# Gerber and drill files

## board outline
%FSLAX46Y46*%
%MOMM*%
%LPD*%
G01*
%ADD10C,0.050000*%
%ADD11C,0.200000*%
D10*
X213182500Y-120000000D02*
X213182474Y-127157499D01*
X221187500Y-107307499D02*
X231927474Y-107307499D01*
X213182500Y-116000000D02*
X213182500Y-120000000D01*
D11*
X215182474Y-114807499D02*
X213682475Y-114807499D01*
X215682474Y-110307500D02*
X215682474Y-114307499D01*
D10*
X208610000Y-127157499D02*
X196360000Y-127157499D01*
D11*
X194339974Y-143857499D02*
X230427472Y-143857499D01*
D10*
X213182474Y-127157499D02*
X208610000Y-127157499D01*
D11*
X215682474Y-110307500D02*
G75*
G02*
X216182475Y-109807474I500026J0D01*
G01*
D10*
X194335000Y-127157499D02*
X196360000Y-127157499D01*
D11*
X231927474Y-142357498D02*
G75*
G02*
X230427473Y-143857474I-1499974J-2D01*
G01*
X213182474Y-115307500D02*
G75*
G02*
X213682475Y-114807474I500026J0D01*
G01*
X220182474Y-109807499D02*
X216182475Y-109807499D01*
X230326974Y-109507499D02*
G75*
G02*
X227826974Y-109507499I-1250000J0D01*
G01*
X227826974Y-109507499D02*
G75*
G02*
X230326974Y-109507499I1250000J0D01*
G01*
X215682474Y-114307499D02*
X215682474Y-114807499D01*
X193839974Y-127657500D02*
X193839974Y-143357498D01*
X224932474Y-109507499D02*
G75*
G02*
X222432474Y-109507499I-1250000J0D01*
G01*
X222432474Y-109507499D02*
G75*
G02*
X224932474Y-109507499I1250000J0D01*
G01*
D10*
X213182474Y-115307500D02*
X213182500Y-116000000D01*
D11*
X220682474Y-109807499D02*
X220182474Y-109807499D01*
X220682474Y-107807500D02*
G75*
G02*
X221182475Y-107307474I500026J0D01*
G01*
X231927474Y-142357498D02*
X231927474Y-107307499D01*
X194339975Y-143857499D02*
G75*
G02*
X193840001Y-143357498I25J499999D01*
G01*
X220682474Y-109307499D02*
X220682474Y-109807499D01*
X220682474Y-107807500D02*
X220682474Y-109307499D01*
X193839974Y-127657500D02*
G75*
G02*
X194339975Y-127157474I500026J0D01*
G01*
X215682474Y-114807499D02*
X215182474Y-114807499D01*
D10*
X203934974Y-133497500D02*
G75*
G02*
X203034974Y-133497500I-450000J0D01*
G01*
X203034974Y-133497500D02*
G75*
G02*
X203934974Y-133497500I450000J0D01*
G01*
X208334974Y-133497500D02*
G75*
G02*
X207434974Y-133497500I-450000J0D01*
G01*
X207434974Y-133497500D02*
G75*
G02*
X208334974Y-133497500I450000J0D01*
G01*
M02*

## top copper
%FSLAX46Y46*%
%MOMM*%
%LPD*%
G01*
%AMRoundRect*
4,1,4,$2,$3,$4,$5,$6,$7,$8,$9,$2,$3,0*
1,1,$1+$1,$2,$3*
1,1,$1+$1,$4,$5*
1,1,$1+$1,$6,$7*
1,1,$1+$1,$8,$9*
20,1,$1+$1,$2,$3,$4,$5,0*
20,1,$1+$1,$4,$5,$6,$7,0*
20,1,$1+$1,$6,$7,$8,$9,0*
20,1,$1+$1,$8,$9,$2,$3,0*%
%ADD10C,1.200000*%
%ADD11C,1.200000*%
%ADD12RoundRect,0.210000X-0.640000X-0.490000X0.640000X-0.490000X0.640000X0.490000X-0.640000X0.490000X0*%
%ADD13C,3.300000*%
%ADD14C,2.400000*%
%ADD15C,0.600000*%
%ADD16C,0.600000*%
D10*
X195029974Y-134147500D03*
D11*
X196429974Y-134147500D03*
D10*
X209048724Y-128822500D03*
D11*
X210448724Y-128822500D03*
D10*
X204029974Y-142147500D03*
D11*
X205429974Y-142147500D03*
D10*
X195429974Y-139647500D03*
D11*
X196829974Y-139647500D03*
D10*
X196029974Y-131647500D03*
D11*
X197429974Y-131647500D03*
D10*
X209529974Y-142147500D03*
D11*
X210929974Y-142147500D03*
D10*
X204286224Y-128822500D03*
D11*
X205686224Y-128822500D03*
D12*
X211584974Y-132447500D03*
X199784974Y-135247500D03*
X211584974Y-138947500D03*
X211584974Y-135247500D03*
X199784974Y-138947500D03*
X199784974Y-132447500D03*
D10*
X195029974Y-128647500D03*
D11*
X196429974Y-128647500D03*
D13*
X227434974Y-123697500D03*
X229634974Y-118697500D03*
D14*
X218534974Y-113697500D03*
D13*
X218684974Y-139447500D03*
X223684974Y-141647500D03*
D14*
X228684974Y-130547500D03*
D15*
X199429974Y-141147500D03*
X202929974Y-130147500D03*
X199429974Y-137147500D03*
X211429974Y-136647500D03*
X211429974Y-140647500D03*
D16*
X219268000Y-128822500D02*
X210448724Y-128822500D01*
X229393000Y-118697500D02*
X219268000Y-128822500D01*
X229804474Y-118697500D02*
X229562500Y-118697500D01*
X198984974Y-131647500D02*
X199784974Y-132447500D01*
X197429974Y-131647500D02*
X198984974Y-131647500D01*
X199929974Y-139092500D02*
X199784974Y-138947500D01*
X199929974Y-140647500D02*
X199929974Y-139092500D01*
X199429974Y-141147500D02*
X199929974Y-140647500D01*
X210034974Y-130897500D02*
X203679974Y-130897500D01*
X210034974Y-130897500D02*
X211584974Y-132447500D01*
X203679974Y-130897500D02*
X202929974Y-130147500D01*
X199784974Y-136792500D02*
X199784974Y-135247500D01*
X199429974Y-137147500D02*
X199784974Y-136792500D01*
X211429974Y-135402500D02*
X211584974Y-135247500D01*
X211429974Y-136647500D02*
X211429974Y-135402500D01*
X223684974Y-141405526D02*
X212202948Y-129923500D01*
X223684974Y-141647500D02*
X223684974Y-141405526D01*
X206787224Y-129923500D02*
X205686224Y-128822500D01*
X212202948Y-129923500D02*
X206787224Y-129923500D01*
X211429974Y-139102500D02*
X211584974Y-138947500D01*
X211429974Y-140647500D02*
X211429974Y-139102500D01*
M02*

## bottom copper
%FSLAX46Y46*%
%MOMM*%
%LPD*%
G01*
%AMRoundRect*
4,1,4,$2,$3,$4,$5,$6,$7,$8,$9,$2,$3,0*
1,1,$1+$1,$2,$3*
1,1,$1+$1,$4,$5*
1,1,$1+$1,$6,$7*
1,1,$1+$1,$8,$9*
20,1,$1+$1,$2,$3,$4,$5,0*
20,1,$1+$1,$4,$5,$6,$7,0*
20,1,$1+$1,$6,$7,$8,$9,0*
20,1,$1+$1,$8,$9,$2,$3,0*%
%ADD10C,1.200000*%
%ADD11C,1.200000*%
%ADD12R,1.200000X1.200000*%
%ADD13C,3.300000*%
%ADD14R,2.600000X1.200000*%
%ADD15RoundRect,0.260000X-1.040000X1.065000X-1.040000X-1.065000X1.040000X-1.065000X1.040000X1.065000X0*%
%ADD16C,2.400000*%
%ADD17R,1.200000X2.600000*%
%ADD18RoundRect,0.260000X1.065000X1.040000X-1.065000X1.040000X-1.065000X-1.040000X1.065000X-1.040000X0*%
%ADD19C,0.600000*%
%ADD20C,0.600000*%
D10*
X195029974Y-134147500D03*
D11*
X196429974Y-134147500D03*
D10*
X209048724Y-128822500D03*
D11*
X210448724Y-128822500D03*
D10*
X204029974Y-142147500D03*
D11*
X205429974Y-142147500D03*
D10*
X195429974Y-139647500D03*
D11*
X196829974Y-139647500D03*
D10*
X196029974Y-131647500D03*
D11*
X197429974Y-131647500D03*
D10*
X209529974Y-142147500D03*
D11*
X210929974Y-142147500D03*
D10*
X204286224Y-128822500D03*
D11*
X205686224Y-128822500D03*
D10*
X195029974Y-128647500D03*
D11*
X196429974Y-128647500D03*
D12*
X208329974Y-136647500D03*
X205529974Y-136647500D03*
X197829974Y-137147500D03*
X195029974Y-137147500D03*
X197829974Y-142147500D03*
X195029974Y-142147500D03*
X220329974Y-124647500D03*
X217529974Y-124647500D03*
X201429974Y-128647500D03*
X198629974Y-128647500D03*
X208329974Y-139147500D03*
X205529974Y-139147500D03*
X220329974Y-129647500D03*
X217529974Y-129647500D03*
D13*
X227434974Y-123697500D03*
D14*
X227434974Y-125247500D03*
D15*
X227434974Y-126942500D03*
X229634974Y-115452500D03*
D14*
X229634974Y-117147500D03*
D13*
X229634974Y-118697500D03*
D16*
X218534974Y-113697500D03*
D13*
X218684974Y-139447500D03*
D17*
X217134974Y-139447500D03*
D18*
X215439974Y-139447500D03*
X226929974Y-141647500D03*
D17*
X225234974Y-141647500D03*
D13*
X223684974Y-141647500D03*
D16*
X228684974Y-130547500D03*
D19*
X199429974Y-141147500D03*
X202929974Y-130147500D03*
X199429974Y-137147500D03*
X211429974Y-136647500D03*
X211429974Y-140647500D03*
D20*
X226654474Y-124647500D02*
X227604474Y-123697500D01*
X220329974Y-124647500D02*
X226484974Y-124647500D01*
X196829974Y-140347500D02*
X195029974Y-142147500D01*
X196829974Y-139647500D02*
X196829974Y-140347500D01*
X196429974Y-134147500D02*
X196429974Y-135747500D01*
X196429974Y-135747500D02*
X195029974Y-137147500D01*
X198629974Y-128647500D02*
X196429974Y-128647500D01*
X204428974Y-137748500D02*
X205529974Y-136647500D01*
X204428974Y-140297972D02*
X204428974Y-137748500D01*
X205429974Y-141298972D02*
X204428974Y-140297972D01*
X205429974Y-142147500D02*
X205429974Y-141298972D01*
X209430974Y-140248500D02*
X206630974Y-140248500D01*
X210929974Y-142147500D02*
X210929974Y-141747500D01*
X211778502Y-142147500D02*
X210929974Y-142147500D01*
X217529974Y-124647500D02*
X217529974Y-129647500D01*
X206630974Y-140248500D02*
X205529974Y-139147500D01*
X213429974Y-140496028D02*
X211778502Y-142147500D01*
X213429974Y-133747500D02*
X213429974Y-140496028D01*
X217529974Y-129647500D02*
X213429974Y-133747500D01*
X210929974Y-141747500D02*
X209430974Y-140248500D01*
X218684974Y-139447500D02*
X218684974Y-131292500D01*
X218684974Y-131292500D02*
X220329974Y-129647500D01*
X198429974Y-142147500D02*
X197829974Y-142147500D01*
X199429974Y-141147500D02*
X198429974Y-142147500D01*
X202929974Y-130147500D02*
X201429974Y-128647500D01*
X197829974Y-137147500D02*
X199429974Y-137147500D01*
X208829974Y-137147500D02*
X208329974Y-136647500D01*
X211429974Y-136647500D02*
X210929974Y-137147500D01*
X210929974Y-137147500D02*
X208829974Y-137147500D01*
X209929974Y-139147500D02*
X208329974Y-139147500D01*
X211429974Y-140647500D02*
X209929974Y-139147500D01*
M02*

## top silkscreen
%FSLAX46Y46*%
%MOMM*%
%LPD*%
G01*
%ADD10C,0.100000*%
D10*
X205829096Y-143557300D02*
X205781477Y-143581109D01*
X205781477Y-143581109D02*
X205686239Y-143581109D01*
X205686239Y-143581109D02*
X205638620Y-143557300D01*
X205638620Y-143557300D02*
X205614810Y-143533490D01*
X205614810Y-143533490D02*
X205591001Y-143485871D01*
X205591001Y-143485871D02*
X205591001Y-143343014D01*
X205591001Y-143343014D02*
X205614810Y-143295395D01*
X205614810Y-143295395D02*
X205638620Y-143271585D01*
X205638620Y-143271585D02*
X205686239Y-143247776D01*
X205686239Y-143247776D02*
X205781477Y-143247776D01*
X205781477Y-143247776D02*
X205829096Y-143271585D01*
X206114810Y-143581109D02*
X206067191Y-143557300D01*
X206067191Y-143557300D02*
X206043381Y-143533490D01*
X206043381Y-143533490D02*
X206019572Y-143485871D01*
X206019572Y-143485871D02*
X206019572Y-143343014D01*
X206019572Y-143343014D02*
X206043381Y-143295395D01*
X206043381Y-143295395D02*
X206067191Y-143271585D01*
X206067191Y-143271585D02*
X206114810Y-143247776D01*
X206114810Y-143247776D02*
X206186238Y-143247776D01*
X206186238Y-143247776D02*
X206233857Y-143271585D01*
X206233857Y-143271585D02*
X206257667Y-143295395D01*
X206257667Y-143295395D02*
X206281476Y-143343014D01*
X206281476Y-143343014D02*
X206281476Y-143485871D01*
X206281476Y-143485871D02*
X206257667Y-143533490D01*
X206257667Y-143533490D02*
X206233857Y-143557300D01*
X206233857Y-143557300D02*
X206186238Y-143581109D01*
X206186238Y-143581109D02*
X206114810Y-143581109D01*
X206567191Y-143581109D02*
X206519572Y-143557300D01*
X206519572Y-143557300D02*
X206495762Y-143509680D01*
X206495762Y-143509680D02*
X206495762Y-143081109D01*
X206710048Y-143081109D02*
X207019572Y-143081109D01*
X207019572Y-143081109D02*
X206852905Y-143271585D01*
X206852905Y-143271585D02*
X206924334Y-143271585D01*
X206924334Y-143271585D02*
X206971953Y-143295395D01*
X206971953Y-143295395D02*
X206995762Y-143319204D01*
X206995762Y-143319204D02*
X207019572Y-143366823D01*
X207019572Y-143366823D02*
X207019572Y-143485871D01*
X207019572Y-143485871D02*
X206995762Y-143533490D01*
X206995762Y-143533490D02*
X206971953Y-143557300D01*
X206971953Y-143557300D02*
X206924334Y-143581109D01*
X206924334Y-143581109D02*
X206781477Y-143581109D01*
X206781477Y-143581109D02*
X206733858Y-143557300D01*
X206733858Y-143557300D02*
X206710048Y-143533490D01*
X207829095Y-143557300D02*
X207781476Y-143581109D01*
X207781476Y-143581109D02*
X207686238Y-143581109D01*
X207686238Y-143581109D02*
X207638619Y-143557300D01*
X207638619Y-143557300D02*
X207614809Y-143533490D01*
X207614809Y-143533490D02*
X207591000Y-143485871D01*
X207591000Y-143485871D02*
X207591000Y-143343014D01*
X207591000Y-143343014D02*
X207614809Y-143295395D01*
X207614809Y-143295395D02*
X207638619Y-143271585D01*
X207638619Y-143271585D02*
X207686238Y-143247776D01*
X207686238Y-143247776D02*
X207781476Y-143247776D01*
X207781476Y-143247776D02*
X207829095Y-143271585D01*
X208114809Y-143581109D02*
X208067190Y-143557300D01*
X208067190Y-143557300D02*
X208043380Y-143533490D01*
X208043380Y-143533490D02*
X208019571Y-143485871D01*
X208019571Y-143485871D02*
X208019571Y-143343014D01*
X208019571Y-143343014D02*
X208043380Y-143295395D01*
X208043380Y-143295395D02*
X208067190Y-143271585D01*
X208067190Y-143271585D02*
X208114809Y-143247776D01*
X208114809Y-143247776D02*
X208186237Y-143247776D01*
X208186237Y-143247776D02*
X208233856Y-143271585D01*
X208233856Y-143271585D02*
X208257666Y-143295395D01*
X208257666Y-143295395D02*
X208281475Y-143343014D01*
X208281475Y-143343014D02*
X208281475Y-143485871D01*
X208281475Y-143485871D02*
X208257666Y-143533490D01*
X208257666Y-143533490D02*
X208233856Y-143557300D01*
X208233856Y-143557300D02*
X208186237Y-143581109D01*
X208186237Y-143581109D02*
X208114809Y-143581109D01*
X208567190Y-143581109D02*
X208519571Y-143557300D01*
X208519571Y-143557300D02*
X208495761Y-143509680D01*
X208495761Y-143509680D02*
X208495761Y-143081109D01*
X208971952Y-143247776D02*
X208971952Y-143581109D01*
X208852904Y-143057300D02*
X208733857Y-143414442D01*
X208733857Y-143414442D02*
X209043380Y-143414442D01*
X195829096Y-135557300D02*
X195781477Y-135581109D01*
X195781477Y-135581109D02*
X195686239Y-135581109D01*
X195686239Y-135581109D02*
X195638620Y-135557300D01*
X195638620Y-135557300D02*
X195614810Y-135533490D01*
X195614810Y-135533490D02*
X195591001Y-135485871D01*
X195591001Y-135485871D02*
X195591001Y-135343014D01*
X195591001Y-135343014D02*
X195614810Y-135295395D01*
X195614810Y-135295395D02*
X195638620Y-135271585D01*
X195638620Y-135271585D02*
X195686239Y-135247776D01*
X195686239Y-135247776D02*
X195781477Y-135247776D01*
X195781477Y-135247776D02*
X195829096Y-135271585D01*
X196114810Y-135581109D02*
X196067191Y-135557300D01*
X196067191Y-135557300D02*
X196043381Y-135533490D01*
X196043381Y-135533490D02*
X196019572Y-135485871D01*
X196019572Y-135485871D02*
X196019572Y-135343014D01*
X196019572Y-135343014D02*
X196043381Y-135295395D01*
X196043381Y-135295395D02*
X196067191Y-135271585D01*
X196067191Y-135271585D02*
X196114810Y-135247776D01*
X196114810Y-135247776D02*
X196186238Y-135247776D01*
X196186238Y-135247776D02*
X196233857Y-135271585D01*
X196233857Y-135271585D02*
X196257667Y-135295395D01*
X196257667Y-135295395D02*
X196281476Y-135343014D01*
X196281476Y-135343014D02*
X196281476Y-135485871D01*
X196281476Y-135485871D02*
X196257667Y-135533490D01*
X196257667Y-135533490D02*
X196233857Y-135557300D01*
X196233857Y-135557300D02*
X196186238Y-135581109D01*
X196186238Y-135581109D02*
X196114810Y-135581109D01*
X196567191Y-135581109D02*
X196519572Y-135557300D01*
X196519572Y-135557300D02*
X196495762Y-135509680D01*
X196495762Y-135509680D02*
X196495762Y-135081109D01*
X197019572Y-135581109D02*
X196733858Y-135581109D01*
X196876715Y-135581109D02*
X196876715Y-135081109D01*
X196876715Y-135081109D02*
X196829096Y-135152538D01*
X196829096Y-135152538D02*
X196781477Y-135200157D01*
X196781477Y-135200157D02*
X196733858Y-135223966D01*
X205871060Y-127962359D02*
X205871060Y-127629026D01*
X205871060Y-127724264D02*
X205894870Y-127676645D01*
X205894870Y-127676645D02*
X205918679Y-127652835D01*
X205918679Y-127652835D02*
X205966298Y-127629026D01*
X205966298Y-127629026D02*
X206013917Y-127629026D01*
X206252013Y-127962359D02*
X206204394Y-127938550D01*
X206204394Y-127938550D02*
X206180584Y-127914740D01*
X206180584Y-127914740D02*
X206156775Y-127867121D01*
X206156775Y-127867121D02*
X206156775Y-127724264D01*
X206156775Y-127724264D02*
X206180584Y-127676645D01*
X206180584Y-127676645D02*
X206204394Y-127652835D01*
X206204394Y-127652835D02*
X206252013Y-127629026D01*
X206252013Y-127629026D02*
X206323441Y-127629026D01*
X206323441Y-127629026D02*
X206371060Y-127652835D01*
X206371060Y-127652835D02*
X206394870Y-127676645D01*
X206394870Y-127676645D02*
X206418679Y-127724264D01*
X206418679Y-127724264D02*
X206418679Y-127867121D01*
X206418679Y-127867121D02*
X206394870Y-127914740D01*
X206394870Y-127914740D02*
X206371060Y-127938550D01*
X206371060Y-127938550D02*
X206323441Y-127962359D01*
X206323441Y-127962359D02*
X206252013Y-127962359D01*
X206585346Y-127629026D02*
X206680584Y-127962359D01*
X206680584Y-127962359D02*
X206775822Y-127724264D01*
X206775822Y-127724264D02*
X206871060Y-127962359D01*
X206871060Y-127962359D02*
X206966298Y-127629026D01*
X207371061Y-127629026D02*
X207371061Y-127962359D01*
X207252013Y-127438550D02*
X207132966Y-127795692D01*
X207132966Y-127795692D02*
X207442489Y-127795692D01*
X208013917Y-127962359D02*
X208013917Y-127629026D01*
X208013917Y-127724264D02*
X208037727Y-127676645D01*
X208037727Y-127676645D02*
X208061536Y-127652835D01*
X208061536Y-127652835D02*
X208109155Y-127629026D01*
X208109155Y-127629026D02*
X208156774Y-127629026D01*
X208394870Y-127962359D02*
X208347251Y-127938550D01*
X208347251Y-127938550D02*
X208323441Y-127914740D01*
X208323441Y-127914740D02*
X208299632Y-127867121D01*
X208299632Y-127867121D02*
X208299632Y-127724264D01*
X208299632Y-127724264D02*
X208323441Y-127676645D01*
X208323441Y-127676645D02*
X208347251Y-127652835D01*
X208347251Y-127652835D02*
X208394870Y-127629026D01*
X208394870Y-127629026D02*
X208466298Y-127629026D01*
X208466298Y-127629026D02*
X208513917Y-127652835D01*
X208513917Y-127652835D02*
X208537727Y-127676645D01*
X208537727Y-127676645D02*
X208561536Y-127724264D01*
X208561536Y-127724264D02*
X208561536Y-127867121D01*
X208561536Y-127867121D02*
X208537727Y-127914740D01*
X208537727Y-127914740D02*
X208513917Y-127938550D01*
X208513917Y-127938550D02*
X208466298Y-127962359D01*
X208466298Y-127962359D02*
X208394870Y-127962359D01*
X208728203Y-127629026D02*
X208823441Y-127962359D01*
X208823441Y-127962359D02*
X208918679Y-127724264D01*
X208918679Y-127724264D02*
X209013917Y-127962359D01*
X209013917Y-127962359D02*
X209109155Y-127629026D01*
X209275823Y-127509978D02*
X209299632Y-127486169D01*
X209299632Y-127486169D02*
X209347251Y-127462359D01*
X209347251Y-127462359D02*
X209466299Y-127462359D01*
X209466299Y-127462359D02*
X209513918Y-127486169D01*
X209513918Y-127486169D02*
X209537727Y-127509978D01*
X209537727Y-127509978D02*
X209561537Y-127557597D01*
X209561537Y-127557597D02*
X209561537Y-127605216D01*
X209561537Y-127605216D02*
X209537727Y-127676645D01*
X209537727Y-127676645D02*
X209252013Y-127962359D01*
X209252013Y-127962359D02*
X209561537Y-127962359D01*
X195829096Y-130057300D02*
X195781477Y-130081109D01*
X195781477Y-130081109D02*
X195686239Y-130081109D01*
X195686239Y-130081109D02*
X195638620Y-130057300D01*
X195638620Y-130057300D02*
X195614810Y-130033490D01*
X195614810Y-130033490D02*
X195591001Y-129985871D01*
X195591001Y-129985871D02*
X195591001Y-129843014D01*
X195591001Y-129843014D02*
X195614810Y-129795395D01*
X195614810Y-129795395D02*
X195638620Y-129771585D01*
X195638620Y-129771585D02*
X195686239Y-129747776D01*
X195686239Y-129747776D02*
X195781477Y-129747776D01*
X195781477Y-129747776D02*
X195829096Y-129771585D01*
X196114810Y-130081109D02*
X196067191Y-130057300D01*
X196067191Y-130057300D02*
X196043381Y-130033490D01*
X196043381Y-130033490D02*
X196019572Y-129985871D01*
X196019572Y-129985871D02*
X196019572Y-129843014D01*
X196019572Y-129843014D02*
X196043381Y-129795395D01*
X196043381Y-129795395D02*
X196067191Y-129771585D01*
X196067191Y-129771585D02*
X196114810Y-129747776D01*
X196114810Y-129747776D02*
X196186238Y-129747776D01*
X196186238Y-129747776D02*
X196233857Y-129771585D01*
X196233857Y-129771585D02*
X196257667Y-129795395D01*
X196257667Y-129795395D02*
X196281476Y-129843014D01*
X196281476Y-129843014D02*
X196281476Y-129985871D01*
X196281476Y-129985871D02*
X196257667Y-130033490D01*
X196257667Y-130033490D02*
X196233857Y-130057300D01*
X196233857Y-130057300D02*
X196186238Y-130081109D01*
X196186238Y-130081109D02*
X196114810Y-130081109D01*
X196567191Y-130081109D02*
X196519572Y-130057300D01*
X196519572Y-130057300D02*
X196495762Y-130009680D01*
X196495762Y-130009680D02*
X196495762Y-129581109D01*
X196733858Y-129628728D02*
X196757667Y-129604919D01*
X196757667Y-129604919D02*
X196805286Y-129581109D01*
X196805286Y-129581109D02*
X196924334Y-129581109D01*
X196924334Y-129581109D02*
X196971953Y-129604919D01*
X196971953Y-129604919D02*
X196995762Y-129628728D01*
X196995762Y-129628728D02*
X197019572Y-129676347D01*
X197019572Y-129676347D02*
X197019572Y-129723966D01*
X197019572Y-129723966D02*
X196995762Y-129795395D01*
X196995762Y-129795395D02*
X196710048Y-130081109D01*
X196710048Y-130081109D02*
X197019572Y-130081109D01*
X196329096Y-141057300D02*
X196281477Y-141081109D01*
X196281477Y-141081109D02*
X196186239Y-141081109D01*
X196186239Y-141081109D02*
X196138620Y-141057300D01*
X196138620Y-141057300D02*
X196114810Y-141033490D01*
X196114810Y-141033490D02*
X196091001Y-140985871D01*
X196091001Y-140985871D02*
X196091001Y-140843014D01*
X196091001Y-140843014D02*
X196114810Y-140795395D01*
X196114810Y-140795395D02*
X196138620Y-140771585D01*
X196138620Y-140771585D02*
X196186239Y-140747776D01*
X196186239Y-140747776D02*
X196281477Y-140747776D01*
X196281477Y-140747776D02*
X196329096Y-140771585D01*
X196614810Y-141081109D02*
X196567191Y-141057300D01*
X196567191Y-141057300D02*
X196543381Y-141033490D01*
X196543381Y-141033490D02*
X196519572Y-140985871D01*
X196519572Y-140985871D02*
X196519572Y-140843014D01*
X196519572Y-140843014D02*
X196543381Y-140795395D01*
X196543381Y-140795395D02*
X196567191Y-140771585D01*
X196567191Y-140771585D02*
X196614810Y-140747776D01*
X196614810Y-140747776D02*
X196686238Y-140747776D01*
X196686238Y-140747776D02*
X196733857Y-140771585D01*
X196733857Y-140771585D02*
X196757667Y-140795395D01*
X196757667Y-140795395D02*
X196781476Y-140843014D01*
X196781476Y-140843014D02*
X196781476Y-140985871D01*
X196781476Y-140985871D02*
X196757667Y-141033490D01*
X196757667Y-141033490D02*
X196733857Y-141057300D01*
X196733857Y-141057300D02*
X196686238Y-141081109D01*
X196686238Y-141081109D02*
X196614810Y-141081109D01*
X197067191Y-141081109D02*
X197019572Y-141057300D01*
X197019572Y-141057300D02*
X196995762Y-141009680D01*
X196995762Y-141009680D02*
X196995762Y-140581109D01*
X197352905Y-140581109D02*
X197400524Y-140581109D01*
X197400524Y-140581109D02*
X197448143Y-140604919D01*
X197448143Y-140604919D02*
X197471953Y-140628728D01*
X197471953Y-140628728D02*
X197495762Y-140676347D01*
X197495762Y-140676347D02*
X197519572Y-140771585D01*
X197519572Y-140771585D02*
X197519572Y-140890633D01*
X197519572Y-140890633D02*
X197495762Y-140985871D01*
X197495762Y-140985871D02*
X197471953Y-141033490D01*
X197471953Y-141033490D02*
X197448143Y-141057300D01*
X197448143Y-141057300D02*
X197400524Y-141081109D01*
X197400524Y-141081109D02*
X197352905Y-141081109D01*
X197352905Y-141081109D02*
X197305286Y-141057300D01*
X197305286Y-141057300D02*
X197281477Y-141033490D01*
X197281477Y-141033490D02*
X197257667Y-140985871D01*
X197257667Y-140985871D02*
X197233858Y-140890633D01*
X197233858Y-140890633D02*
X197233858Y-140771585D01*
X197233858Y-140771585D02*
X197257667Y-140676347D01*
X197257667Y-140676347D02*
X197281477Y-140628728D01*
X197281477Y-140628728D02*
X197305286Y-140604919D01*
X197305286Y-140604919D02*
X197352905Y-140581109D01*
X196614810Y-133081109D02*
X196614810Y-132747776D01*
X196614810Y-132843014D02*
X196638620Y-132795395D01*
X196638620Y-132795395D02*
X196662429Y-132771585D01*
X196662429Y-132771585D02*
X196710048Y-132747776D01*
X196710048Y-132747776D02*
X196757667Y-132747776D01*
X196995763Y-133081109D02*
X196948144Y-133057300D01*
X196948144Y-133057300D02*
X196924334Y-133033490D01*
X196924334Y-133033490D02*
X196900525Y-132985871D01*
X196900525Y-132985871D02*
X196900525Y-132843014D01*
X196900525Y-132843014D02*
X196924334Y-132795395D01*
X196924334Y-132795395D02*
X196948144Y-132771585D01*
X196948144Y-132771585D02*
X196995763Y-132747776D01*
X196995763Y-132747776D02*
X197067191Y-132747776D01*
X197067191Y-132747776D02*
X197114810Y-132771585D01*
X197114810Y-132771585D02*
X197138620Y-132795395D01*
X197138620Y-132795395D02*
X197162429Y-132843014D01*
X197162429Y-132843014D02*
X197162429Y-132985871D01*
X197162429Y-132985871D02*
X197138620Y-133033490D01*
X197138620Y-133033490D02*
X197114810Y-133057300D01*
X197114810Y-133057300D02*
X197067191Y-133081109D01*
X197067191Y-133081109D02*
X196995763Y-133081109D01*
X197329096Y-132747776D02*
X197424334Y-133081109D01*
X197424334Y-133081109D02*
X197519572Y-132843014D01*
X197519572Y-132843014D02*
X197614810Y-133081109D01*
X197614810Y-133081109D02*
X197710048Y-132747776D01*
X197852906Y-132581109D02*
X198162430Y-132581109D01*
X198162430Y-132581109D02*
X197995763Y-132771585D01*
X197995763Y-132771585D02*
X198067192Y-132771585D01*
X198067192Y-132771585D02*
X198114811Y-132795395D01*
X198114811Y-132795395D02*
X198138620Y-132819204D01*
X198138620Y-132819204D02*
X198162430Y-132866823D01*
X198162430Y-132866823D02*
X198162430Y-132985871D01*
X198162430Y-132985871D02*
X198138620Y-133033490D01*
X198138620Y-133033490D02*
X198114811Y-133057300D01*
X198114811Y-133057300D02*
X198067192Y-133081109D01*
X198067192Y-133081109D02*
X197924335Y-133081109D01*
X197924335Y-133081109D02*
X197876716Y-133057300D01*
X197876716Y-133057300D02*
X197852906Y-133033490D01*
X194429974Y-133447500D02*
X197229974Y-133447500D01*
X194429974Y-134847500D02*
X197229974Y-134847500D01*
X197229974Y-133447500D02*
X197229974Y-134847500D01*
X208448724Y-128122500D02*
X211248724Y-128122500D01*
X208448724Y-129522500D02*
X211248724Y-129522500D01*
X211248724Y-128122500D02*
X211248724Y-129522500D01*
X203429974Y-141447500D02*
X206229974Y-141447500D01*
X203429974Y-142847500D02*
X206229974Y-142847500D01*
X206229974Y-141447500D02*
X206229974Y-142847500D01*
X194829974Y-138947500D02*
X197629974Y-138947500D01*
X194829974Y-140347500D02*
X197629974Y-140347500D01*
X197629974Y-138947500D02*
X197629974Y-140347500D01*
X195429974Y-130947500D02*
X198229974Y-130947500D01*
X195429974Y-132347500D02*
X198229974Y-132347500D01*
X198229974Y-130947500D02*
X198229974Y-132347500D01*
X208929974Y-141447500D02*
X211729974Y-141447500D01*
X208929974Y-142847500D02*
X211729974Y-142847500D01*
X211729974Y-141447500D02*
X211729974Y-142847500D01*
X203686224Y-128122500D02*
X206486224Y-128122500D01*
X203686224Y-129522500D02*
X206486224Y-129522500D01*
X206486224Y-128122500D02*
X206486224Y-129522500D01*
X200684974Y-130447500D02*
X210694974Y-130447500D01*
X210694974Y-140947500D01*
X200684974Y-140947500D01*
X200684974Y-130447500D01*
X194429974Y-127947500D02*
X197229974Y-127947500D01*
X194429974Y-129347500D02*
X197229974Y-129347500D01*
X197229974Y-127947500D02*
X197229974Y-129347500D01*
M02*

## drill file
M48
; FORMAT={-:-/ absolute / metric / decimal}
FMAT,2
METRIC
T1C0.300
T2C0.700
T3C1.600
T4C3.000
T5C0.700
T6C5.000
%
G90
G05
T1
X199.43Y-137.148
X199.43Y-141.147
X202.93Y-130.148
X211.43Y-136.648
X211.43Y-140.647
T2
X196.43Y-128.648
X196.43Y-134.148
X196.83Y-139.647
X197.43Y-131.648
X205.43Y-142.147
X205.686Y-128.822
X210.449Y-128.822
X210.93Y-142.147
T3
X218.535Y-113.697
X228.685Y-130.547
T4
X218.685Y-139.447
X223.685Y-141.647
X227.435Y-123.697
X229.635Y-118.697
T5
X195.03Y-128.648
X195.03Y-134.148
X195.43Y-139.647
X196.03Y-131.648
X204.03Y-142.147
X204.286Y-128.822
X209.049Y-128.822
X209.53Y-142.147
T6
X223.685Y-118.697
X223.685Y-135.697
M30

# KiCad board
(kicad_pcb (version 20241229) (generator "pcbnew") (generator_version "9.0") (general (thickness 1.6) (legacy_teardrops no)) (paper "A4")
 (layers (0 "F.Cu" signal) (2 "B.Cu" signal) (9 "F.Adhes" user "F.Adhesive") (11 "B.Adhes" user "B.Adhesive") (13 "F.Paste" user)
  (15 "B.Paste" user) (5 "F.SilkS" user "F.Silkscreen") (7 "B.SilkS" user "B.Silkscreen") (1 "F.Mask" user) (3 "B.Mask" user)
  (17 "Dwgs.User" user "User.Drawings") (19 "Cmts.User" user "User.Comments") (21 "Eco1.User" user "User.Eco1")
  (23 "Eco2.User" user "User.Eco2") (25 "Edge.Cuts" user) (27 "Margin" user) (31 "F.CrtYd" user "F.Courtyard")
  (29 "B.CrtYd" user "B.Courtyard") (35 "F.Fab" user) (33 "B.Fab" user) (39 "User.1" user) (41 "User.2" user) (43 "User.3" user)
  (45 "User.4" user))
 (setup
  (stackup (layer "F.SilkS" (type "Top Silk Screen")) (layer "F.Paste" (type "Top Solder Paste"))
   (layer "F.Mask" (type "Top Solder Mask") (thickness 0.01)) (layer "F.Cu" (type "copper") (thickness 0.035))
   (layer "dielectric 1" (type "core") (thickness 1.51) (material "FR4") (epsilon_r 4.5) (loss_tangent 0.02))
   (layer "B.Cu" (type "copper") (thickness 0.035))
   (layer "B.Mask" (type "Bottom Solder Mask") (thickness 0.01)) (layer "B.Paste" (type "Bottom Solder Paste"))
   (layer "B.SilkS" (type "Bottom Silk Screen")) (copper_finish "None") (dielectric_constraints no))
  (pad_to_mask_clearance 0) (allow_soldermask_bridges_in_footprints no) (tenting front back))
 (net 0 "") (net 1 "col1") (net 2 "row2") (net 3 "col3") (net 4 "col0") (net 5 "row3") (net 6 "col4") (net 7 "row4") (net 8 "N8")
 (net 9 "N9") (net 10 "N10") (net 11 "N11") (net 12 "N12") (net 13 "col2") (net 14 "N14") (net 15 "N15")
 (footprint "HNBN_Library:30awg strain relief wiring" (layer "F.Cu") (at 196.429974 134.1475)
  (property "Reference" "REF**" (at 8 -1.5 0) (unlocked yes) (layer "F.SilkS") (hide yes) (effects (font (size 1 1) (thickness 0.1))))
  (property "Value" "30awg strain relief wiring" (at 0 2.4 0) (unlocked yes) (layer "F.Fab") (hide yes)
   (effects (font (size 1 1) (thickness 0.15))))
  (fp_line (start -2 -0.7) (end 0.8 -0.7) (stroke (width 0.1) (type default)) (layer "F.SilkS"))
  (fp_line (start -2 0.7) (end 0.8 0.7) (stroke (width 0.1) (type default)) (layer "F.SilkS"))
  (fp_line (start 0.8 -0.7) (end 0.8 0.7) (stroke (width 0.1) (type default)) (layer "F.SilkS"))
  (pad "" np_thru_hole circle (at -1.4 0) (size 1.2 1.2) (drill 0.7) (layers "*.Cu" "*.Mask")
   (teardrops (best_length_ratio 0.5) (max_length 1) (best_width_ratio 0.6) (max_width 2) (curved_edges no) (filter_ratio 0.9) (enabled no)
    (allow_two_segments yes) (prefer_zone_connections yes)))
  (pad "1" thru_hole circle (at 0 0) (size 1.2 1.2) (drill 0.7) (layers "*.Cu" "*.Mask") (remove_unused_layers no) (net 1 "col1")))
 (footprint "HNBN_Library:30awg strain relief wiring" (layer "F.Cu") (at 210.448724 128.8225)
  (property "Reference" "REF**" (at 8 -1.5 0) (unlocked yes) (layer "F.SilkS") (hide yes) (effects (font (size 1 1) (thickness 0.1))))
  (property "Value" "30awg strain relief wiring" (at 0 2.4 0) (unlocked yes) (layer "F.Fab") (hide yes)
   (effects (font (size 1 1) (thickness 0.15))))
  (fp_line (start -2 -0.7) (end 0.8 -0.7) (stroke (width 0.1) (type default)) (layer "F.SilkS"))
  (fp_line (start -2 0.7) (end 0.8 0.7) (stroke (width 0.1) (type default)) (layer "F.SilkS"))
  (fp_line (start 0.8 -0.7) (end 0.8 0.7) (stroke (width 0.1) (type default)) (layer "F.SilkS"))
  (pad "" np_thru_hole circle (at -1.4 0) (size 1.2 1.2) (drill 0.7) (layers "*.Cu" "*.Mask")
   (teardrops (best_length_ratio 0.5) (max_length 1) (best_width_ratio 0.6) (max_width 2) (curved_edges no) (filter_ratio 0.9) (enabled no)
    (allow_two_segments yes) (prefer_zone_connections yes)))
  (pad "1" thru_hole circle (at 0 0) (size 1.2 1.2) (drill 0.7) (layers "*.Cu" "*.Mask") (remove_unused_layers no) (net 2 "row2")))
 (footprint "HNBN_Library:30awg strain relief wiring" (layer "F.Cu") (at 205.429974 142.1475)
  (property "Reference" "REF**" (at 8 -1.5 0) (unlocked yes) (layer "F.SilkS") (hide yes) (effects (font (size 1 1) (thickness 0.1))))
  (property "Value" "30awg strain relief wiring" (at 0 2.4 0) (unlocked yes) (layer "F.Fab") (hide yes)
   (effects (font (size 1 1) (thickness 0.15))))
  (fp_line (start -2 -0.7) (end 0.8 -0.7) (stroke (width 0.1) (type default)) (layer "F.SilkS"))
  (fp_line (start -2 0.7) (end 0.8 0.7) (stroke (width 0.1) (type default)) (layer "F.SilkS"))
  (fp_line (start 0.8 -0.7) (end 0.8 0.7) (stroke (width 0.1) (type default)) (layer "F.SilkS"))
  (pad "" np_thru_hole circle (at -1.4 0) (size 1.2 1.2) (drill 0.7) (layers "*.Cu" "*.Mask")
   (teardrops (best_length_ratio 0.5) (max_length 1) (best_width_ratio 0.6) (max_width 2) (curved_edges no) (filter_ratio 0.9) (enabled no)
    (allow_two_segments yes) (prefer_zone_connections yes)))
  (pad "1" thru_hole circle (at 0 0) (size 1.2 1.2) (drill 0.7) (layers "*.Cu" "*.Mask") (remove_unused_layers no) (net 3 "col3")))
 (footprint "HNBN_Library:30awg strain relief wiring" (layer "F.Cu") (at 196.829974 139.6475)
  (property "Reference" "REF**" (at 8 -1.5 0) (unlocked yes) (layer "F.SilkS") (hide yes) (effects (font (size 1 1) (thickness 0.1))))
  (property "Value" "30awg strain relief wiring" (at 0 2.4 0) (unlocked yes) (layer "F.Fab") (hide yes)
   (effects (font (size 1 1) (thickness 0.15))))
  (fp_line (start -2 -0.7) (end 0.8 -0.7) (stroke (width 0.1) (type default)) (layer "F.SilkS"))
  (fp_line (start -2 0.7) (end 0.8 0.7) (stroke (width 0.1) (type default)) (layer "F.SilkS"))
  (fp_line (start 0.8 -0.7) (end 0.8 0.7) (stroke (width 0.1) (type default)) (layer "F.SilkS"))
  (pad "" np_thru_hole circle (at -1.4 0) (size 1.2 1.2) (drill 0.7) (layers "*.Cu" "*.Mask")
   (teardrops (best_length_ratio 0.5) (max_length 1) (best_width_ratio 0.6) (max_width 2) (curved_edges no) (filter_ratio 0.9) (enabled no)
    (allow_two_segments yes) (prefer_zone_connections yes)))
  (pad "1" thru_hole circle (at 0 0) (size 1.2 1.2) (drill 0.7) (layers "*.Cu" "*.Mask") (remove_unused_layers no) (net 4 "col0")))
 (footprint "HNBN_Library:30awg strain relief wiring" (layer "F.Cu") (at 197.429974 131.6475)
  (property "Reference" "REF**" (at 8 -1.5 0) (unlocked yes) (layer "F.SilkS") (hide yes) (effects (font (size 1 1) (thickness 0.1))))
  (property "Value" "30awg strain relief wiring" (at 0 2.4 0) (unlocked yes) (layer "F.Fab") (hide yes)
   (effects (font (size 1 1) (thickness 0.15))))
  (fp_line (start -2 -0.7) (end 0.8 -0.7) (stroke (width 0.1) (type default)) (layer "F.SilkS"))
  (fp_line (start -2 0.7) (end 0.8 0.7) (stroke (width 0.1) (type default)) (layer "F.SilkS"))
  (fp_line (start 0.8 -0.7) (end 0.8 0.7) (stroke (width 0.1) (type default)) (layer "F.SilkS"))
  (pad "" np_thru_hole circle (at -1.4 0) (size 1.2 1.2) (drill 0.7) (layers "*.Cu" "*.Mask")
   (teardrops (best_length_ratio 0.5) (max_length 1) (best_width_ratio 0.6) (max_width 2) (curved_edges no) (filter_ratio 0.9) (enabled no)
    (allow_two_segments yes) (prefer_zone_connections yes)))
  (pad "1" thru_hole circle (at 0 0) (size 1.2 1.2) (drill 0.7) (layers "*.Cu" "*.Mask") (remove_unused_layers no) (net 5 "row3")))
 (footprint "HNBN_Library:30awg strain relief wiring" (layer "F.Cu") (at 210.929974 142.1475)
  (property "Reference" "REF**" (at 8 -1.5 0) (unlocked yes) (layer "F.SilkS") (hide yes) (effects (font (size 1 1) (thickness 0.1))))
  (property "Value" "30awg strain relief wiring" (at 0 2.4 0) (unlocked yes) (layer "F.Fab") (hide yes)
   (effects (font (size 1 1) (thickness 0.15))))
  (fp_line (start -2 -0.7) (end 0.8 -0.7) (stroke (width 0.1) (type default)) (layer "F.SilkS"))
  (fp_line (start -2 0.7) (end 0.8 0.7) (stroke (width 0.1) (type default)) (layer "F.SilkS"))
  (fp_line (start 0.8 -0.7) (end 0.8 0.7) (stroke (width 0.1) (type default)) (layer "F.SilkS"))
  (pad "" np_thru_hole circle (at -1.4 0) (size 1.2 1.2) (drill 0.7) (layers "*.Cu" "*.Mask")
   (teardrops (best_length_ratio 0.5) (max_length 1) (best_width_ratio 0.6) (max_width 2) (curved_edges no) (filter_ratio 0.9) (enabled no)
    (allow_two_segments yes) (prefer_zone_connections yes)))
  (pad "1" thru_hole circle (at 0 0) (size 1.2 1.2) (drill 0.7) (layers "*.Cu" "*.Mask") (remove_unused_layers no) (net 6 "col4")))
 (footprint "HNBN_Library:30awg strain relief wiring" (layer "F.Cu") (at 205.686224 128.8225)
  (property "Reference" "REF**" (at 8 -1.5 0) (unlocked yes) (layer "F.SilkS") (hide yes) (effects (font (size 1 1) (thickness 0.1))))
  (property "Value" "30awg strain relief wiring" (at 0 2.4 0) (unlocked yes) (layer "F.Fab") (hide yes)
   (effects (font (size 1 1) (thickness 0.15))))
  (fp_line (start -2 -0.7) (end 0.8 -0.7) (stroke (width 0.1) (type default)) (layer "F.SilkS"))
  (fp_line (start -2 0.7) (end 0.8 0.7) (stroke (width 0.1) (type default)) (layer "F.SilkS"))
  (fp_line (start 0.8 -0.7) (end 0.8 0.7) (stroke (width 0.1) (type default)) (layer "F.SilkS"))
  (pad "" np_thru_hole circle (at -1.4 0) (size 1.2 1.2) (drill 0.7) (layers "*.Cu" "*.Mask")
   (teardrops (best_length_ratio 0.5) (max_length 1) (best_width_ratio 0.6) (max_width 2) (curved_edges no) (filter_ratio 0.9) (enabled no)
    (allow_two_segments yes) (prefer_zone_connections yes)))
  (pad "1" thru_hole circle (at 0 0) (size 1.2 1.2) (drill 0.7) (layers "*.Cu" "*.Mask") (remove_unused_layers no) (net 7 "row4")))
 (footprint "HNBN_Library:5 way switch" (layer "F.Cu") (at 205.684974 135.6975)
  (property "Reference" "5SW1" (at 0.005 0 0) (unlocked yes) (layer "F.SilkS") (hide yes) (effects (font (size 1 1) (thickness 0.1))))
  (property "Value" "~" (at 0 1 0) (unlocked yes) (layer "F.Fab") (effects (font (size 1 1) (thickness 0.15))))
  (fp_rect (start -5 -5.25) (end 5.01 5.25) (stroke (width 0.1) (type default)) (fill no) (layer "F.SilkS"))
  (fp_circle (center -2.2 -2.2) (end -1.75 -2.2) (stroke (width 0.05) (type default)) (fill no) (layer "Edge.Cuts"))
  (fp_circle (center 2.2 -2.2) (end 2.65 -2.2) (stroke (width 0.05) (type default)) (fill no) (layer "Edge.Cuts"))
  (pad "F1" smd roundrect (at 5.9 -3.25) (size 1.7 1.4) (layers "F.Cu" "F.Mask" "F.Paste") (roundrect_rratio 0.15) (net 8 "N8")
   (thermal_bridge_angle 45))
  (pad "F2" smd roundrect (at -5.9 -0.45) (size 1.7 1.4) (layers "F.Cu" "F.Mask" "F.Paste") (roundrect_rratio 0.15) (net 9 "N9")
   (thermal_bridge_angle 45))
  (pad "F3" smd roundrect (at 5.9 3.25) (size 1.7 1.4) (layers "F.Cu" "F.Mask" "F.Paste") (roundrect_rratio 0.15) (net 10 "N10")
   (thermal_bridge_angle 45))
  (pad "F4" smd roundrect (at 5.9 -0.45) (size 1.7 1.4) (layers "F.Cu" "F.Mask" "F.Paste") (roundrect_rratio 0.15) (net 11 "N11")
   (thermal_bridge_angle 45))
  (pad "F5" smd roundrect (at -5.9 3.25) (size 1.7 1.4) (layers "F.Cu" "F.Mask" "F.Paste") (roundrect_rratio 0.15) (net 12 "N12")
   (thermal_bridge_angle 45))
  (pad "com" smd roundrect (at -5.9 -3.25) (size 1.7 1.4) (layers "F.Cu" "F.Mask" "F.Paste") (roundrect_rratio 0.15) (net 5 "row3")
   (thermal_bridge_angle 45)))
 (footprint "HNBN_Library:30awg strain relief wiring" (layer "F.Cu") (at 196.429974 128.6475)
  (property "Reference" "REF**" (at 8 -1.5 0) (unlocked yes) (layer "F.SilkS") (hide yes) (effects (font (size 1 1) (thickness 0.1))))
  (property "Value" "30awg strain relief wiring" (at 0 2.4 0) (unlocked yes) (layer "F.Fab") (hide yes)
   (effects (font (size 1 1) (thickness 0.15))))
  (fp_line (start -2 -0.7) (end 0.8 -0.7) (stroke (width 0.1) (type default)) (layer "F.SilkS"))
  (fp_line (start -2 0.7) (end 0.8 0.7) (stroke (width 0.1) (type default)) (layer "F.SilkS"))
  (fp_line (start 0.8 -0.7) (end 0.8 0.7) (stroke (width 0.1) (type default)) (layer "F.SilkS"))
  (pad "" np_thru_hole circle (at -1.4 0) (size 1.2 1.2) (drill 0.7) (layers "*.Cu" "*.Mask")
   (teardrops (best_length_ratio 0.5) (max_length 1) (best_width_ratio 0.6) (max_width 2) (curved_edges no) (filter_ratio 0.9) (enabled no)
    (allow_two_segments yes) (prefer_zone_connections yes)))
  (pad "1" thru_hole circle (at 0 0) (size 1.2 1.2) (drill 0.7) (layers "*.Cu" "*.Mask") (remove_unused_layers no) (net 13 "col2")))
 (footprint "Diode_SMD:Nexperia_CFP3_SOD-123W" (layer "B.Cu") (at 206.929974 136.6475 180)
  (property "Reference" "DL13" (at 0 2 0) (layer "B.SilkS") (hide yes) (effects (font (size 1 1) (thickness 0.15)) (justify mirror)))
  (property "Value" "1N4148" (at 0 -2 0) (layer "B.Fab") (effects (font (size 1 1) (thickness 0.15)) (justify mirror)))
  (pad "1" smd rect (at -1.4 0 180) (size 1.2 1.2) (layers "B.Cu" "B.Mask" "B.Paste") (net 11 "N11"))
  (pad "2" smd rect (at 1.4 0 180) (size 1.2 1.2) (layers "B.Cu" "B.Mask" "B.Paste") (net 3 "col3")))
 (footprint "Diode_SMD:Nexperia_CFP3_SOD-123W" (layer "B.Cu") (at 196.429974 137.1475 180)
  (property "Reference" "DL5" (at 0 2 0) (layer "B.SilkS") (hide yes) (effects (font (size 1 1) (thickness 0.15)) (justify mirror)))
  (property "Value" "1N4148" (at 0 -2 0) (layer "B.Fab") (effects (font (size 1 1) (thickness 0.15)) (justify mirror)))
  (pad "1" smd rect (at -1.4 0 180) (size 1.2 1.2) (layers "B.Cu" "B.Mask" "B.Paste") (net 9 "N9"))
  (pad "2" smd rect (at 1.4 0 180) (size 1.2 1.2) (layers "B.Cu" "B.Mask" "B.Paste") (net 1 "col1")))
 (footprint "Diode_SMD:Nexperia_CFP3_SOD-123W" (layer "B.Cu") (at 196.429974 142.1475 180)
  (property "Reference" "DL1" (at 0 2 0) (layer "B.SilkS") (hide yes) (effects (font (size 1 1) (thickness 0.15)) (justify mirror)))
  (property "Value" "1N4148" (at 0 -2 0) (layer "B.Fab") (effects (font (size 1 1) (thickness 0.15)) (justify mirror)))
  (pad "1" smd rect (at -1.4 0 180) (size 1.2 1.2) (layers "B.Cu" "B.Mask" "B.Paste") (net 12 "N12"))
  (pad "2" smd rect (at 1.4 0 180) (size 1.2 1.2) (layers "B.Cu" "B.Mask" "B.Paste") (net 4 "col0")))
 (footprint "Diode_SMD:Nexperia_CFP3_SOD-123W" (layer "B.Cu") (at 218.929974 124.6475 180)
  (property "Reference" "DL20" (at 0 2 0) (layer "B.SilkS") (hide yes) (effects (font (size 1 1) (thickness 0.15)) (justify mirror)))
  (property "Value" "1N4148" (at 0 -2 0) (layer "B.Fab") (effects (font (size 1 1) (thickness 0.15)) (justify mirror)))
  (pad "1" smd rect (at -1.4 0 180) (size 1.2 1.2) (layers "B.Cu" "B.Mask" "B.Paste") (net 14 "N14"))
  (pad "2" smd rect (at 1.4 0 180) (size 1.2 1.2) (layers "B.Cu" "B.Mask" "B.Paste") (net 6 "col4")))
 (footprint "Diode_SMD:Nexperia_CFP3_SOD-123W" (layer "B.Cu") (at 200.029974 128.6475 180)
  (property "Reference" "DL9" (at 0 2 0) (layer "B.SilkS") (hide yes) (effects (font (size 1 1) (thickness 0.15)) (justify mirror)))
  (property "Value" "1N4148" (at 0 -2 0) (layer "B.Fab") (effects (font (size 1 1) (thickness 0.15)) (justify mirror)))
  (pad "1" smd rect (at -1.4 0 180) (size 1.2 1.2) (layers "B.Cu" "B.Mask" "B.Paste") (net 8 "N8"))
  (pad "2" smd rect (at 1.4 0 180) (size 1.2 1.2) (layers "B.Cu" "B.Mask" "B.Paste") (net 13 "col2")))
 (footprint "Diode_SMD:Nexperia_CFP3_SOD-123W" (layer "B.Cu") (at 206.929974 139.1475 180)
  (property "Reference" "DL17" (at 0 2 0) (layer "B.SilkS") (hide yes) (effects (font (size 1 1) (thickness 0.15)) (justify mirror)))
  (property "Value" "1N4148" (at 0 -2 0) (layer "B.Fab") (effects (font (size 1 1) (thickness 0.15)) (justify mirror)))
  (pad "1" smd rect (at -1.4 0 180) (size 1.2 1.2) (layers "B.Cu" "B.Mask" "B.Paste") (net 10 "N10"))
  (pad "2" smd rect (at 1.4 0 180) (size 1.2 1.2) (layers "B.Cu" "B.Mask" "B.Paste") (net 6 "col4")))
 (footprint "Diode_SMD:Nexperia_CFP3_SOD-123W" (layer "B.Cu") (at 218.929974 129.6475 180)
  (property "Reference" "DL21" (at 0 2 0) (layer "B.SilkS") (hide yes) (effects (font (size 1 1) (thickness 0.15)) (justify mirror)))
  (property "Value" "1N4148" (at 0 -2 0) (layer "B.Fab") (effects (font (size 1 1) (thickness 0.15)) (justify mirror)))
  (pad "1" smd rect (at -1.4 0 180) (size 1.2 1.2) (layers "B.Cu" "B.Mask" "B.Paste") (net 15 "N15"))
  (pad "2" smd rect (at 1.4 0 180) (size 1.2 1.2) (layers "B.Cu" "B.Mask" "B.Paste") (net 6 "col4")))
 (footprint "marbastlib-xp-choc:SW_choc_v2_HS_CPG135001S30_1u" (layer "B.Cu") (at 223.684974 118.6975 -90)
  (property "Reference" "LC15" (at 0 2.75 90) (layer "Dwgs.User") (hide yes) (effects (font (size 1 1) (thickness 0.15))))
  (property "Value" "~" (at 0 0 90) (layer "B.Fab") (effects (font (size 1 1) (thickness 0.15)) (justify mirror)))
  (pad "" np_thru_hole circle (at 0 0 90) (size 5 5) (drill 5) (layers "*.Cu" "*.Mask"))
  (pad "1" thru_hole circle (at 5 -3.75 270) (size 3.3 3.3) (drill 3) (layers "*.Cu" "B.Mask") (remove_unused_layers no) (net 14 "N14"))
  (pad "1" smd rect (at 6.55 -3.75 270) (size 1.2 2.6) (layers "B.Cu") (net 14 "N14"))
  (pad "1" smd roundrect (at 8.245 -3.75 270) (size 2.65 2.6) (layers "B.Cu" "B.Mask" "B.Paste") (roundrect_rratio 0.1) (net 14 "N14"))
  (pad "2" smd roundrect (at -3.245 -5.95 270) (size 2.65 2.6) (layers "B.Cu" "B.Mask" "B.Paste") (roundrect_rratio 0.1) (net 2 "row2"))
  (pad "2" smd rect (at -1.55 -5.95 90) (size 1.2 2.6) (layers "B.Cu") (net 2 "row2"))
  (pad "2" thru_hole circle (at 0 -5.95 270) (size 3.3 3.3) (drill 3) (layers "*.Cu" "B.Mask") (remove_unused_layers no) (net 2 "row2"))
  (pad "MP" thru_hole circle (at -5 5.15 90) (size 2.4 2.4) (drill 1.6) (layers "*.Cu" "B.Mask") (remove_unused_layers no)))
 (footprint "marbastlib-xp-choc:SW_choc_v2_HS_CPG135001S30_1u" (layer "B.Cu") (at 223.684974 135.6975 180)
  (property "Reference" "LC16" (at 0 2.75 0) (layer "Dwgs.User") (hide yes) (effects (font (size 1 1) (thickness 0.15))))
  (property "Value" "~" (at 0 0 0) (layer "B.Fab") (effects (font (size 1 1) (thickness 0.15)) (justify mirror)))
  (pad "" np_thru_hole circle (at 0 0) (size 5 5) (drill 5) (layers "*.Cu" "*.Mask"))
  (pad "1" thru_hole circle (at 5 -3.75 180) (size 3.3 3.3) (drill 3) (layers "*.Cu" "B.Mask") (remove_unused_layers no) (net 15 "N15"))
  (pad "1" smd rect (at 6.55 -3.75 180) (size 1.2 2.6) (layers "B.Cu") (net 15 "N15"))
  (pad "1" smd roundrect (at 8.245 -3.75 180) (size 2.65 2.6) (layers "B.Cu" "B.Mask" "B.Paste") (roundrect_rratio 0.1) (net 15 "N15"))
  (pad "2" smd roundrect (at -3.245 -5.95 180) (size 2.65 2.6) (layers "B.Cu" "B.Mask" "B.Paste") (roundrect_rratio 0.1) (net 7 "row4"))
  (pad "2" smd rect (at -1.55 -5.95) (size 1.2 2.6) (layers "B.Cu") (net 7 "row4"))
  (pad "2" thru_hole circle (at 0 -5.95 180) (size 3.3 3.3) (drill 3) (layers "*.Cu" "B.Mask") (remove_unused_layers no) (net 7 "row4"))
  (pad "MP" thru_hole circle (at -5 5.15) (size 2.4 2.4) (drill 1.6) (layers "*.Cu" "B.Mask") (remove_unused_layers no)))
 (gr_line (start 213.1825 120) (end 213.182474 127.157499) (stroke (width 0.05) (type default)) (layer "Edge.Cuts"))
 (gr_line (start 221.1875 107.307499) (end 231.927474 107.307499) (stroke (width 0.05) (type default)) (layer "Edge.Cuts"))
 (gr_line (start 213.1825 116) (end 213.1825 120) (stroke (width 0.05) (type default)) (layer "Edge.Cuts"))
 (gr_line (start 215.182474 114.807499) (end 213.682475 114.807499) (stroke (width 0.2) (type default)) (layer "Edge.Cuts"))
 (gr_line (start 215.682474 110.3075) (end 215.682474 114.307499) (stroke (width 0.2) (type default)) (layer "Edge.Cuts"))
 (gr_line (start 208.61 127.157499) (end 196.36 127.157499) (stroke (width 0.05) (type default)) (layer "Edge.Cuts"))
 (gr_line (start 194.339974 143.857499) (end 230.427472 143.857499) (stroke (width 0.2) (type default)) (layer "Edge.Cuts"))
 (gr_line (start 213.182474 127.157499) (end 208.61 127.157499) (stroke (width 0.05) (type default)) (layer "Edge.Cuts"))
 (gr_arc (start 215.682474 110.3075) (mid 215.828921 109.953946) (end 216.182475 109.807499) (stroke (width 0.2) (type default))
  (layer "Edge.Cuts"))
 (gr_line (start 194.335 127.157499) (end 196.36 127.157499) (stroke (width 0.05) (type default)) (layer "Edge.Cuts"))
 (gr_arc (start 231.927474 142.357498) (mid 231.488134 143.418159) (end 230.427473 143.857499) (stroke (width 0.2) (type default))
  (layer "Edge.Cuts"))
 (gr_arc (start 213.182474 115.3075) (mid 213.328921 114.953946) (end 213.682475 114.807499) (stroke (width 0.2) (type default))
  (layer "Edge.Cuts"))
 (gr_line (start 220.182474 109.807499) (end 216.182475 109.807499) (stroke (width 0.2) (type default)) (layer "Edge.Cuts"))
 (gr_circle (center 229.076974 109.507499) (end 227.826974 109.507499) (stroke (width 0.2) (type default)) (fill no) (layer "Edge.Cuts"))
 (gr_line (start 215.682474 114.307499) (end 215.682474 114.807499) (stroke (width 0.2) (type default)) (layer "Edge.Cuts"))
 (gr_line (start 193.839974 127.6575) (end 193.839974 143.357498) (stroke (width 0.2) (type default)) (layer "Edge.Cuts"))
 (gr_circle (center 223.682474 109.507499) (end 222.432474 109.507499) (stroke (width 0.2) (type default)) (fill no) (layer "Edge.Cuts"))
 (gr_line (start 213.182474 115.3075) (end 213.1825 116) (stroke (width 0.05) (type default)) (layer "Edge.Cuts"))
 (gr_line (start 220.682474 109.807499) (end 220.182474 109.807499) (stroke (width 0.2) (type default)) (layer "Edge.Cuts"))
 (gr_arc (start 220.682474 107.8075) (mid 220.828921 107.453946) (end 221.182475 107.307499) (stroke (width 0.2) (type default))
  (layer "Edge.Cuts"))
 (gr_line (start 231.927474 142.357498) (end 231.927474 107.307499) (stroke (width 0.2) (type default)) (layer "Edge.Cuts"))
 (gr_arc (start 194.339975 143.857499) (mid 193.986421 143.711052) (end 193.839974 143.357498) (stroke (width 0.2) (type default))
  (layer "Edge.Cuts"))
 (gr_line (start 220.682474 109.307499) (end 220.682474 109.807499) (stroke (width 0.2) (type default)) (layer "Edge.Cuts"))
 (gr_line (start 220.682474 107.8075) (end 220.682474 109.307499) (stroke (width 0.2) (type default)) (layer "Edge.Cuts"))
 (gr_arc (start 193.839974 127.6575) (mid 193.986421 127.303946) (end 194.339975 127.157499) (stroke (width 0.2) (type default))
  (layer "Edge.Cuts"))
 (gr_line (start 215.682474 114.807499) (end 215.182474 114.807499) (stroke (width 0.2) (type default)) (layer "Edge.Cuts"))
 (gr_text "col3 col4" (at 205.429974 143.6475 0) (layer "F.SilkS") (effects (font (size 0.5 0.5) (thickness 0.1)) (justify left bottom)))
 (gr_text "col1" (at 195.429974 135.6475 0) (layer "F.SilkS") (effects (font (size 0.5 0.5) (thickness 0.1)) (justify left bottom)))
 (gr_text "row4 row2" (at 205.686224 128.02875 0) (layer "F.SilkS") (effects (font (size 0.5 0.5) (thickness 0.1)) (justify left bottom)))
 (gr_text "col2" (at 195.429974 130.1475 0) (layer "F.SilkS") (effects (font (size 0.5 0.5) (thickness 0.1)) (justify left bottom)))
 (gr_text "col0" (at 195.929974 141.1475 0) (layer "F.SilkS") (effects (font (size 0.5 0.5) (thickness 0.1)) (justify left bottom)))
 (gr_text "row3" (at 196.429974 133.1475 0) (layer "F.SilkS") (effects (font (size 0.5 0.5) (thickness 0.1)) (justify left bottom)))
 (segment (start 226.654474 124.6475) (end 227.604474 123.6975) (width 0.6) (layer "B.Cu") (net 14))
 (segment (start 220.329974 124.6475) (end 226.484974 124.6475) (width 0.6) (layer "B.Cu") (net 14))
 (segment (start 219.268 128.8225) (end 210.448724 128.8225) (width 0.6) (layer "F.Cu") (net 2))
 (segment (start 229.393 118.6975) (end 219.268 128.8225) (width 0.6) (layer "F.Cu") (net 2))
 (segment (start 229.804474 118.6975) (end 229.5625 118.6975) (width 0.6) (layer "F.Cu") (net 2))
 (segment (start 198.984974 131.6475) (end 199.784974 132.4475) (width 0.6) (layer "F.Cu") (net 5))
 (segment (start 197.429974 131.6475) (end 198.984974 131.6475) (width 0.6) (layer "F.Cu") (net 5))
 (segment (start 196.829974 140.3475) (end 195.029974 142.1475) (width 0.6) (layer "B.Cu") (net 4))
 (segment (start 196.829974 139.6475) (end 196.829974 140.3475) (width 0.6) (layer "B.Cu") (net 4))
 (segment (start 196.429974 134.1475) (end 196.429974 135.7475) (width 0.6) (layer "B.Cu") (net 1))
 (segment (start 196.429974 135.7475) (end 195.029974 137.1475) (width 0.6) (layer "B.Cu") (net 1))
 (segment (start 198.629974 128.6475) (end 196.429974 128.6475) (width 0.6) (layer "B.Cu") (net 13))
 (segment (start 204.428974 137.7485) (end 205.529974 136.6475) (width 0.6) (layer "B.Cu") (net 3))
 (segment (start 204.428974 140.297972) (end 204.428974 137.7485) (width 0.6) (layer "B.Cu") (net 3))
 (segment (start 205.429974 141.298972) (end 204.428974 140.297972) (width 0.6) (layer "B.Cu") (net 3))
 (segment (start 205.429974 142.1475) (end 205.429974 141.298972) (width 0.6) (layer "B.Cu") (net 3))
 (segment (start 209.430974 140.2485) (end 206.630974 140.2485) (width 0.6) (layer "B.Cu") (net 6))
 (segment (start 210.929974 142.1475) (end 210.929974 141.7475) (width 0.6) (layer "B.Cu") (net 6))
 (segment (start 211.778502 142.1475) (end 210.929974 142.1475) (width 0.6) (layer "B.Cu") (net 6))
 (segment (start 217.529974 124.6475) (end 217.529974 129.6475) (width 0.6) (layer "B.Cu") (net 6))
 (segment (start 206.630974 140.2485) (end 205.529974 139.1475) (width 0.6) (layer "B.Cu") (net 6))
 (segment (start 213.429974 140.496028) (end 211.778502 142.1475) (width 0.6) (layer "B.Cu") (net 6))
 (segment (start 213.429974 133.7475) (end 213.429974 140.496028) (width 0.6) (layer "B.Cu") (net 6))
 (segment (start 217.529974 129.6475) (end 213.429974 133.7475) (width 0.6) (layer "B.Cu") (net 6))
 (segment (start 210.929974 141.7475) (end 209.430974 140.2485) (width 0.6) (layer "B.Cu") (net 6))
 (segment (start 218.684974 139.4475) (end 218.684974 131.2925) (width 0.6) (layer "B.Cu") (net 15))
 (segment (start 218.684974 131.2925) (end 220.329974 129.6475) (width 0.6) (layer "B.Cu") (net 15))
 (segment (start 199.929974 139.0925) (end 199.784974 138.9475) (width 0.6) (layer "F.Cu") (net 12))
 (segment (start 199.929974 140.6475) (end 199.929974 139.0925) (width 0.6) (layer "F.Cu") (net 12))
 (segment (start 199.429974 141.1475) (end 199.929974 140.6475) (width 0.6) (layer "F.Cu") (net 12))
 (via (at 199.429974 141.1475) (size 0.6) (drill 0.3) (layers "F.Cu" "B.Cu") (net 12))
 (segment (start 198.429974 142.1475) (end 197.829974 142.1475) (width 0.6) (layer "B.Cu") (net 12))
 (segment (start 199.429974 141.1475) (end 198.429974 142.1475) (width 0.6) (layer "B.Cu") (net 12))
 (segment (start 210.034974 130.8975) (end 203.679974 130.8975) (width 0.6) (layer "F.Cu") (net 8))
 (segment (start 210.034974 130.8975) (end 211.584974 132.4475) (width 0.6) (layer "F.Cu") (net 8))
 (segment (start 203.679974 130.8975) (end 202.929974 130.1475) (width 0.6) (layer "F.Cu") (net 8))
 (via (at 202.929974 130.1475) (size 0.6) (drill 0.3) (layers "F.Cu" "B.Cu") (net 8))
 (segment (start 202.929974 130.1475) (end 201.429974 128.6475) (width 0.6) (layer "B.Cu") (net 8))
 (segment (start 199.784974 136.7925) (end 199.784974 135.2475) (width 0.6) (layer "F.Cu") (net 9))
 (segment (start 199.429974 137.1475) (end 199.784974 136.7925) (width 0.6) (layer "F.Cu") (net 9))
 (via (at 199.429974 137.1475) (size 0.6) (drill 0.3) (layers "F.Cu" "B.Cu") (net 9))
 (segment (start 197.829974 137.1475) (end 199.429974 137.1475) (width 0.6) (layer "B.Cu") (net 9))
 (segment (start 211.429974 135.4025) (end 211.584974 135.2475) (width 0.6) (layer "F.Cu") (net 11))
 (segment (start 211.429974 136.6475) (end 211.429974 135.4025) (width 0.6) (layer "F.Cu") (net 11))
 (via (at 211.429974 136.6475) (size 0.6) (drill 0.3) (layers "F.Cu" "B.Cu") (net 11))
 (segment (start 208.829974 137.1475) (end 208.329974 136.6475) (width 0.6) (layer "B.Cu") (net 11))
 (segment (start 211.429974 136.6475) (end 210.929974 137.1475) (width 0.6) (layer "B.Cu") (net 11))
 (segment (start 210.929974 137.1475) (end 208.829974 137.1475) (width 0.6) (layer "B.Cu") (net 11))
 (segment (start 223.684974 141.405526) (end 212.202948 129.9235) (width 0.6) (layer "F.Cu") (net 7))
 (segment (start 223.684974 141.6475) (end 223.684974 141.405526) (width 0.6) (layer "F.Cu") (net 7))
 (segment (start 206.787224 129.9235) (end 205.686224 128.8225) (width 0.6) (layer "F.Cu") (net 7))
 (segment (start 212.202948 129.9235) (end 206.787224 129.9235) (width 0.6) (layer "F.Cu") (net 7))
 (segment (start 211.429974 139.1025) (end 211.584974 138.9475) (width 0.6) (layer "F.Cu") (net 10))
 (segment (start 211.429974 140.6475) (end 211.429974 139.1025) (width 0.6) (layer "F.Cu") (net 10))
 (via (at 211.429974 140.6475) (size 0.6) (drill 0.3) (layers "F.Cu" "B.Cu") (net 10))
 (segment (start 209.929974 139.1475) (end 208.329974 139.1475) (width 0.6) (layer "B.Cu") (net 10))
 (segment (start 211.429974 140.6475) (end 209.929974 139.1475) (width 0.6) (layer "B.Cu") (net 10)))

